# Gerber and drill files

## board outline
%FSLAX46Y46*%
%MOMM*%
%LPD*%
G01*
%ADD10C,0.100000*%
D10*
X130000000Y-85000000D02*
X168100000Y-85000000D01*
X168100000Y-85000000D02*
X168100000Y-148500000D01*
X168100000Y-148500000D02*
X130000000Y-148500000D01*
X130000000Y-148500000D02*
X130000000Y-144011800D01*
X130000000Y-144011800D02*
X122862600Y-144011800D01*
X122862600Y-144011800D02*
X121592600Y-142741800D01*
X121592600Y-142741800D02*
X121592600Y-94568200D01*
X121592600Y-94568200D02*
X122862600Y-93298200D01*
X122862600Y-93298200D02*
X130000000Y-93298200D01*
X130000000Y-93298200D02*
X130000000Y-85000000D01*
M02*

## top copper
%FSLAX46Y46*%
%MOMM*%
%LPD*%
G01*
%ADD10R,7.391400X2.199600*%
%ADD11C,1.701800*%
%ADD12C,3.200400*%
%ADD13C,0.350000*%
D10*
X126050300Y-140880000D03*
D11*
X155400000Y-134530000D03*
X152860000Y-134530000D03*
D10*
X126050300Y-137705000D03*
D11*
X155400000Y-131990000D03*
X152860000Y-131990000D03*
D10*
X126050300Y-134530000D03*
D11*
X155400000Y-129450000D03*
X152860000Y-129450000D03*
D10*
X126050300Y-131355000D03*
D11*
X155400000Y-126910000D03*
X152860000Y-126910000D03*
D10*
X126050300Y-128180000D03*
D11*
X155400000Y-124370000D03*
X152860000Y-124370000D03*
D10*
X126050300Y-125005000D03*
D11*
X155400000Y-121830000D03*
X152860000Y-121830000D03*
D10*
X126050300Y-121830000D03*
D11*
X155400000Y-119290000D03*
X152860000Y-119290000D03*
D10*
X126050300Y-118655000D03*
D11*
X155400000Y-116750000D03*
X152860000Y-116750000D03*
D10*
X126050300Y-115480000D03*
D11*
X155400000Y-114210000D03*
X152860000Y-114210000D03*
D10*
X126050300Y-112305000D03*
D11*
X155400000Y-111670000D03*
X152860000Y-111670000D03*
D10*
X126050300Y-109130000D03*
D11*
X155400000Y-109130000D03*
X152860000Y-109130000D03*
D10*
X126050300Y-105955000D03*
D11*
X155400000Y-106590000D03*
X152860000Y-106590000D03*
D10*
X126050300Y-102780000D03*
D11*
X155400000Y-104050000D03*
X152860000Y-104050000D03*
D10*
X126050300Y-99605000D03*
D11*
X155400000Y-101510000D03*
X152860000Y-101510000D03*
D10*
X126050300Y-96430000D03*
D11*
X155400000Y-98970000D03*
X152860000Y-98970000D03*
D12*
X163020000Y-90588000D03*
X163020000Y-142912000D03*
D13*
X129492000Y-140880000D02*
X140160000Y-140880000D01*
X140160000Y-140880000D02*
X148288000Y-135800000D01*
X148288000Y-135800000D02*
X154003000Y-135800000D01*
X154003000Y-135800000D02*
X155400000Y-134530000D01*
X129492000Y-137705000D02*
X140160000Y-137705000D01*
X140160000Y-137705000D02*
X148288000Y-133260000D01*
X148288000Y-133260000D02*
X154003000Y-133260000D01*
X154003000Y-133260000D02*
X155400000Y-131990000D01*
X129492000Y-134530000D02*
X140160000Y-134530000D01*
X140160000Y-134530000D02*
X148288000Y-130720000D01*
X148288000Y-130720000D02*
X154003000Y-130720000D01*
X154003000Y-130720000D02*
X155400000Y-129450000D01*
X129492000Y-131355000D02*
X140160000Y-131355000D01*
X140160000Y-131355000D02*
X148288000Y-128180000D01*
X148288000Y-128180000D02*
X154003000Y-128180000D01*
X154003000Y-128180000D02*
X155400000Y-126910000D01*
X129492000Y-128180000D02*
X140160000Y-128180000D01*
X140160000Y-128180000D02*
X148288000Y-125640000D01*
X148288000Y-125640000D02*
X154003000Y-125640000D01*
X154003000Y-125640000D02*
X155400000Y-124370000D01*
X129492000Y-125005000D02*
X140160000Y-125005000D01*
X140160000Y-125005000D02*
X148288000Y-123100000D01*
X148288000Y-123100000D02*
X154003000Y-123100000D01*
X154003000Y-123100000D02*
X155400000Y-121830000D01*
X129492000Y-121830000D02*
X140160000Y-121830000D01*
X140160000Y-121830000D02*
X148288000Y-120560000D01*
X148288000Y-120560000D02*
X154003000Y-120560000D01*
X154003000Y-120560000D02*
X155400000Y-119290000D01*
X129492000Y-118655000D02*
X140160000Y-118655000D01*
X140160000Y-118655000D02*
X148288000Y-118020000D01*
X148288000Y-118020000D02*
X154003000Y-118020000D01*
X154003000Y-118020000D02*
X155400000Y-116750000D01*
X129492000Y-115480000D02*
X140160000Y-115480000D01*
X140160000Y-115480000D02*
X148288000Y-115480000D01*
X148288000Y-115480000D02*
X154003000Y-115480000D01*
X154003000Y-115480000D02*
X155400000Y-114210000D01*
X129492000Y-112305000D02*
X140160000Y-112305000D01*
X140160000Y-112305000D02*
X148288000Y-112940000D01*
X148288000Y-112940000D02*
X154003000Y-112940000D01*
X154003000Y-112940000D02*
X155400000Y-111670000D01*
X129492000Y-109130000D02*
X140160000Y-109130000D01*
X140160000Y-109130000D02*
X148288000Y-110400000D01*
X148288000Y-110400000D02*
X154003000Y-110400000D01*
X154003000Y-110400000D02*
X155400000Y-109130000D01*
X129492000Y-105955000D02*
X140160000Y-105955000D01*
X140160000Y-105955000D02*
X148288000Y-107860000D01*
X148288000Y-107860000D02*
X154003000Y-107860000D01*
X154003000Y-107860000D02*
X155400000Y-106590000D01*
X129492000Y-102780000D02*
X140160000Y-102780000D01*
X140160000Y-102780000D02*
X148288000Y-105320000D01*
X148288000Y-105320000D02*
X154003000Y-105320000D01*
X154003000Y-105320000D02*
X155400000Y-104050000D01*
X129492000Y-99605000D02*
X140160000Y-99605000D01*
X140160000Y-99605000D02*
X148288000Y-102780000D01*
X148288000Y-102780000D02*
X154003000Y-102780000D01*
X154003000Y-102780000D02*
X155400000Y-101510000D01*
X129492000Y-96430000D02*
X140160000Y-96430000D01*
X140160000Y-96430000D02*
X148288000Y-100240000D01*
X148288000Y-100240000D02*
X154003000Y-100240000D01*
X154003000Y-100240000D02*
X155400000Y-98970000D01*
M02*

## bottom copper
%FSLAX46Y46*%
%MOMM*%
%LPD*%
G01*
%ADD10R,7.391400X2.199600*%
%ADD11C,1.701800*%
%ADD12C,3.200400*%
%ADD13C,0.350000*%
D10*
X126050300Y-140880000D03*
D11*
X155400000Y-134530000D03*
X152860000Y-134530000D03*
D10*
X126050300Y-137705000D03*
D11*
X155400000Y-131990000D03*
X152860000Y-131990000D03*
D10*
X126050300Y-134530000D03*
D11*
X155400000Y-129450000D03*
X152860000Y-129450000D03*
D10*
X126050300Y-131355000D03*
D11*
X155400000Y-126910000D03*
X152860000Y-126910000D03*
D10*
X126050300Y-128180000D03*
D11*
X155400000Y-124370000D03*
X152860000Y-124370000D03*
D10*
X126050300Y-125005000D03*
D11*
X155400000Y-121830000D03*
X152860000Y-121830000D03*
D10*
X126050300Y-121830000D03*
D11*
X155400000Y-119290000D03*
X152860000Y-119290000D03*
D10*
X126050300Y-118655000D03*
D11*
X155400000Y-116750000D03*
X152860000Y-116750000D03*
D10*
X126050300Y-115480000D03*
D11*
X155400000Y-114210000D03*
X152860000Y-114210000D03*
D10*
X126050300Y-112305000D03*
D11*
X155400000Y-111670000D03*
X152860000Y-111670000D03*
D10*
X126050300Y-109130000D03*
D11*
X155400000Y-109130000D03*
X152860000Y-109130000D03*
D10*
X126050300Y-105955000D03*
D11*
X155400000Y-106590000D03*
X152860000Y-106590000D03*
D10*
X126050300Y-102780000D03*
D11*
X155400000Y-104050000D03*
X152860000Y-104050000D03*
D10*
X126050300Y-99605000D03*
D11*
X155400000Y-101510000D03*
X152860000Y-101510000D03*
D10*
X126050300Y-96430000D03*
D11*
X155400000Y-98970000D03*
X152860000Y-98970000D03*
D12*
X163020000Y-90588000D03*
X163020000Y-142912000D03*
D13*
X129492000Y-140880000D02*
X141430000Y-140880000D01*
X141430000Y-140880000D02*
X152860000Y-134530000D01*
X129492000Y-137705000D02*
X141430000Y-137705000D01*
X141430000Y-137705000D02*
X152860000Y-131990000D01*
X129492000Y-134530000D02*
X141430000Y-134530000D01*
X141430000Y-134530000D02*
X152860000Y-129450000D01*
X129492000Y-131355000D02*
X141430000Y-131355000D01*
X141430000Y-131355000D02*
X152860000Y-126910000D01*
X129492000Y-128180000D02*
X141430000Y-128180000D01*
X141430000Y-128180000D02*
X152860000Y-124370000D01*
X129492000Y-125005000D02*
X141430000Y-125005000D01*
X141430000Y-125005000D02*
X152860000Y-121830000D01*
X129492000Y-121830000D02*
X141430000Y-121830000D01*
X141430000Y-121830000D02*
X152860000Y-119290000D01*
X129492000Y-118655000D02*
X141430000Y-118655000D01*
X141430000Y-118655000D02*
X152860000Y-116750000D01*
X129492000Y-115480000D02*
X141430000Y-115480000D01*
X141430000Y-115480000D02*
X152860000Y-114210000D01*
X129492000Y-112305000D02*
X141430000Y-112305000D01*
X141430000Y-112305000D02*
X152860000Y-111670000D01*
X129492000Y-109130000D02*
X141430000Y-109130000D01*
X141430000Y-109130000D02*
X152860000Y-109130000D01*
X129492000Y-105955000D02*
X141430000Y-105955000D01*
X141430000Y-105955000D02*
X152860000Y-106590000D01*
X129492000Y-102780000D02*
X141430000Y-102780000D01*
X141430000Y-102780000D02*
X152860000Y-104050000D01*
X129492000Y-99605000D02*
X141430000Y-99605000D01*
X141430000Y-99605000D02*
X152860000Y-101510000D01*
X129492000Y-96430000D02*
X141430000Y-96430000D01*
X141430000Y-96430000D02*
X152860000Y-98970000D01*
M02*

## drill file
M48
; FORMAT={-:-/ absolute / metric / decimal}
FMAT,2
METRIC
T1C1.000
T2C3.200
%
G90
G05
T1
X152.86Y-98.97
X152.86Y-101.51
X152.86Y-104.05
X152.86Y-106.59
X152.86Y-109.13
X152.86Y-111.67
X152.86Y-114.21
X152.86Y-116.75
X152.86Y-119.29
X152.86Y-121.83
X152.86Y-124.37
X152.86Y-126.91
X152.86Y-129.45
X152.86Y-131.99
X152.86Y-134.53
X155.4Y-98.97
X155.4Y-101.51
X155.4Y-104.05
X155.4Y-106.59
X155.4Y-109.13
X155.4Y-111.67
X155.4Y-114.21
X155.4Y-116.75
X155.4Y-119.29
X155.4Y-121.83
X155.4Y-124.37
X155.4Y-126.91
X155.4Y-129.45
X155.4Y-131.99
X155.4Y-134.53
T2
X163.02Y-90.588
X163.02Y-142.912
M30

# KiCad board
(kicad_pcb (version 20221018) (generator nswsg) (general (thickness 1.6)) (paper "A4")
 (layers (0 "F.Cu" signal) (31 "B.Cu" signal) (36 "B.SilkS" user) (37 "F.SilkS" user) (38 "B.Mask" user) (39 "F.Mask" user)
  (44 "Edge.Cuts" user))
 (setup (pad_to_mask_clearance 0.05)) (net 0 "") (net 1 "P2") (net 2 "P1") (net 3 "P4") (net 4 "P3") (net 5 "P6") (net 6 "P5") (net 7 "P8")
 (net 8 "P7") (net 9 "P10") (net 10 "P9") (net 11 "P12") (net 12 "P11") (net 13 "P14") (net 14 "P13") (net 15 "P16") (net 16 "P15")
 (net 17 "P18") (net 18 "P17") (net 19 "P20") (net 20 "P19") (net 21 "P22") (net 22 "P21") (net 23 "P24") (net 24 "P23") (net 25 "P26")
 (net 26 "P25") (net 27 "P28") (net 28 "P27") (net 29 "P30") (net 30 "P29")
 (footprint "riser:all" (layer "F.Cu") (at 130.0 85.0)
  (pad "2" smd rect (at -3.9497 55.88) (size 7.3914 2.1996) (layers "F.Cu" "F.Mask") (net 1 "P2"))
  (pad "1" smd rect (at -3.9497 55.88) (size 7.3914 2.1996) (layers "B.Cu" "B.Mask") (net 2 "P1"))
  (pad "2" thru_hole circle (at 25.4 49.53) (size 1.7018 1.7018) (drill 1.0) (layers "*.Cu" "*.Mask") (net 1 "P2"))
  (pad "1" thru_hole circle (at 22.86 49.53) (size 1.7018 1.7018) (drill 1.0) (layers "*.Cu" "*.Mask") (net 2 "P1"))
  (pad "4" smd rect (at -3.9497 52.705) (size 7.3914 2.1996) (layers "F.Cu" "F.Mask") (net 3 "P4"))
  (pad "3" smd rect (at -3.9497 52.705) (size 7.3914 2.1996) (layers "B.Cu" "B.Mask") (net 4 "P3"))
  (pad "4" thru_hole circle (at 25.4 46.99) (size 1.7018 1.7018) (drill 1.0) (layers "*.Cu" "*.Mask") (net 3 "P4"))
  (pad "3" thru_hole circle (at 22.86 46.99) (size 1.7018 1.7018) (drill 1.0) (layers "*.Cu" "*.Mask") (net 4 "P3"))
  (pad "6" smd rect (at -3.9497 49.53) (size 7.3914 2.1996) (layers "F.Cu" "F.Mask") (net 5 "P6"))
  (pad "5" smd rect (at -3.9497 49.53) (size 7.3914 2.1996) (layers "B.Cu" "B.Mask") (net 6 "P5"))
  (pad "6" thru_hole circle (at 25.4 44.45) (size 1.7018 1.7018) (drill 1.0) (layers "*.Cu" "*.Mask") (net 5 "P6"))
  (pad "5" thru_hole circle (at 22.86 44.45) (size 1.7018 1.7018) (drill 1.0) (layers "*.Cu" "*.Mask") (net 6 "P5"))
  (pad "8" smd rect (at -3.9497 46.355) (size 7.3914 2.1996) (layers "F.Cu" "F.Mask") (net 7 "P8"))
  (pad "7" smd rect (at -3.9497 46.355) (size 7.3914 2.1996) (layers "B.Cu" "B.Mask") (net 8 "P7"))
  (pad "8" thru_hole circle (at 25.4 41.91) (size 1.7018 1.7018) (drill 1.0) (layers "*.Cu" "*.Mask") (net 7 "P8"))
  (pad "7" thru_hole circle (at 22.86 41.91) (size 1.7018 1.7018) (drill 1.0) (layers "*.Cu" "*.Mask") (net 8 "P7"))
  (pad "10" smd rect (at -3.9497 43.18) (size 7.3914 2.1996) (layers "F.Cu" "F.Mask") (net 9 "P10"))
  (pad "9" smd rect (at -3.9497 43.18) (size 7.3914 2.1996) (layers "B.Cu" "B.Mask") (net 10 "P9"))
  (pad "10" thru_hole circle (at 25.4 39.37) (size 1.7018 1.7018) (drill 1.0) (layers "*.Cu" "*.Mask") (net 9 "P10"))
  (pad "9" thru_hole circle (at 22.86 39.37) (size 1.7018 1.7018) (drill 1.0) (layers "*.Cu" "*.Mask") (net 10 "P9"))
  (pad "12" smd rect (at -3.9497 40.005) (size 7.3914 2.1996) (layers "F.Cu" "F.Mask") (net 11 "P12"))
  (pad "11" smd rect (at -3.9497 40.005) (size 7.3914 2.1996) (layers "B.Cu" "B.Mask") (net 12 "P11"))
  (pad "12" thru_hole circle (at 25.4 36.83) (size 1.7018 1.7018) (drill 1.0) (layers "*.Cu" "*.Mask") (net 11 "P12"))
  (pad "11" thru_hole circle (at 22.86 36.83) (size 1.7018 1.7018) (drill 1.0) (layers "*.Cu" "*.Mask") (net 12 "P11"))
  (pad "14" smd rect (at -3.9497 36.83) (size 7.3914 2.1996) (layers "F.Cu" "F.Mask") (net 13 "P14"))
  (pad "13" smd rect (at -3.9497 36.83) (size 7.3914 2.1996) (layers "B.Cu" "B.Mask") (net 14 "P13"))
  (pad "14" thru_hole circle (at 25.4 34.29) (size 1.7018 1.7018) (drill 1.0) (layers "*.Cu" "*.Mask") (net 13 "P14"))
  (pad "13" thru_hole circle (at 22.86 34.29) (size 1.7018 1.7018) (drill 1.0) (layers "*.Cu" "*.Mask") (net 14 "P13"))
  (pad "16" smd rect (at -3.9497 33.655) (size 7.3914 2.1996) (layers "F.Cu" "F.Mask") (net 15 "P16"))
  (pad "15" smd rect (at -3.9497 33.655) (size 7.3914 2.1996) (layers "B.Cu" "B.Mask") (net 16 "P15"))
  (pad "16" thru_hole circle (at 25.4 31.75) (size 1.7018 1.7018) (drill 1.0) (layers "*.Cu" "*.Mask") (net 15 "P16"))
  (pad "15" thru_hole circle (at 22.86 31.75) (size 1.7018 1.7018) (drill 1.0) (layers "*.Cu" "*.Mask") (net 16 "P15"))
  (pad "18" smd rect (at -3.9497 30.48) (size 7.3914 2.1996) (layers "F.Cu" "F.Mask") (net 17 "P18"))
  (pad "17" smd rect (at -3.9497 30.48) (size 7.3914 2.1996) (layers "B.Cu" "B.Mask") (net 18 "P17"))
  (pad "18" thru_hole circle (at 25.4 29.21) (size 1.7018 1.7018) (drill 1.0) (layers "*.Cu" "*.Mask") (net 17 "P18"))
  (pad "17" thru_hole circle (at 22.86 29.21) (size 1.7018 1.7018) (drill 1.0) (layers "*.Cu" "*.Mask") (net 18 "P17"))
  (pad "20" smd rect (at -3.9497 27.305) (size 7.3914 2.1996) (layers "F.Cu" "F.Mask") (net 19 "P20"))
  (pad "19" smd rect (at -3.9497 27.305) (size 7.3914 2.1996) (layers "B.Cu" "B.Mask") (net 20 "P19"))
  (pad "20" thru_hole circle (at 25.4 26.67) (size 1.7018 1.7018) (drill 1.0) (layers "*.Cu" "*.Mask") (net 19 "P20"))
  (pad "19" thru_hole circle (at 22.86 26.67) (size 1.7018 1.7018) (drill 1.0) (layers "*.Cu" "*.Mask") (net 20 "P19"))
  (pad "22" smd rect (at -3.9497 24.13) (size 7.3914 2.1996) (layers "F.Cu" "F.Mask") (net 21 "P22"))
  (pad "21" smd rect (at -3.9497 24.13) (size 7.3914 2.1996) (layers "B.Cu" "B.Mask") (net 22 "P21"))
  (pad "22" thru_hole circle (at 25.4 24.13) (size 1.7018 1.7018) (drill 1.0) (layers "*.Cu" "*.Mask") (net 21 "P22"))
  (pad "21" thru_hole circle (at 22.86 24.13) (size 1.7018 1.7018) (drill 1.0) (layers "*.Cu" "*.Mask") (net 22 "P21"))
  (pad "24" smd rect (at -3.9497 20.955) (size 7.3914 2.1996) (layers "F.Cu" "F.Mask") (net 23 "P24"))
  (pad "23" smd rect (at -3.9497 20.955) (size 7.3914 2.1996) (layers "B.Cu" "B.Mask") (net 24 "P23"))
  (pad "24" thru_hole circle (at 25.4 21.59) (size 1.7018 1.7018) (drill 1.0) (layers "*.Cu" "*.Mask") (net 23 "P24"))
  (pad "23" thru_hole circle (at 22.86 21.59) (size 1.7018 1.7018) (drill 1.0) (layers "*.Cu" "*.Mask") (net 24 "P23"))
  (pad "26" smd rect (at -3.9497 17.78) (size 7.3914 2.1996) (layers "F.Cu" "F.Mask") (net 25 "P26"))
  (pad "25" smd rect (at -3.9497 17.78) (size 7.3914 2.1996) (layers "B.Cu" "B.Mask") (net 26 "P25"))
  (pad "26" thru_hole circle (at 25.4 19.05) (size 1.7018 1.7018) (drill 1.0) (layers "*.Cu" "*.Mask") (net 25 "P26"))
  (pad "25" thru_hole circle (at 22.86 19.05) (size 1.7018 1.7018) (drill 1.0) (layers "*.Cu" "*.Mask") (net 26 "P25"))
  (pad "28" smd rect (at -3.9497 14.605) (size 7.3914 2.1996) (layers "F.Cu" "F.Mask") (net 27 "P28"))
  (pad "27" smd rect (at -3.9497 14.605) (size 7.3914 2.1996) (layers "B.Cu" "B.Mask") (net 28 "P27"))
  (pad "28" thru_hole circle (at 25.4 16.51) (size 1.7018 1.7018) (drill 1.0) (layers "*.Cu" "*.Mask") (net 27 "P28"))
  (pad "27" thru_hole circle (at 22.86 16.51) (size 1.7018 1.7018) (drill 1.0) (layers "*.Cu" "*.Mask") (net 28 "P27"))
  (pad "30" smd rect (at -3.9497 11.43) (size 7.3914 2.1996) (layers "F.Cu" "F.Mask") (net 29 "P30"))
  (pad "29" smd rect (at -3.9497 11.43) (size 7.3914 2.1996) (layers "B.Cu" "B.Mask") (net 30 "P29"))
  (pad "30" thru_hole circle (at 25.4 13.97) (size 1.7018 1.7018) (drill 1.0) (layers "*.Cu" "*.Mask") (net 29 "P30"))
  (pad "29" thru_hole circle (at 22.86 13.97) (size 1.7018 1.7018) (drill 1.0) (layers "*.Cu" "*.Mask") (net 30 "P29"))
  (pad "" np_thru_hole circle (at 33.02 5.588) (size 3.2004 3.2004) (drill 3.2) (layers "*.Cu" "*.Mask"))
  (pad "" np_thru_hole circle (at 33.02 57.912) (size 3.2004 3.2004) (drill 3.2) (layers "*.Cu" "*.Mask")))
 (gr_line (start 130.0000 85.0000) (end 168.1000 85.0000) (layer "Edge.Cuts") (width 0.1))
 (gr_line (start 168.1000 85.0000) (end 168.1000 148.5000) (layer "Edge.Cuts") (width 0.1))
 (gr_line (start 168.1000 148.5000) (end 130.0000 148.5000) (layer "Edge.Cuts") (width 0.1))
 (gr_line (start 130.0000 148.5000) (end 130.0000 144.0118) (layer "Edge.Cuts") (width 0.1))
 (gr_line (start 130.0000 144.0118) (end 122.8626 144.0118) (layer "Edge.Cuts") (width 0.1))
 (gr_line (start 122.8626 144.0118) (end 121.5926 142.7418) (layer "Edge.Cuts") (width 0.1))
 (gr_line (start 121.5926 142.7418) (end 121.5926 94.5682) (layer "Edge.Cuts") (width 0.1))
 (gr_line (start 121.5926 94.5682) (end 122.8626 93.2982) (layer "Edge.Cuts") (width 0.1))
 (gr_line (start 122.8626 93.2982) (end 130.0000 93.2982) (layer "Edge.Cuts") (width 0.1))
 (gr_line (start 130.0000 93.2982) (end 130.0000 85.0000) (layer "Edge.Cuts") (width 0.1))
 (segment (start 129.4920 140.8800) (end 140.1600 140.8800) (width 0.35) (layer "F.Cu") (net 1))
 (segment (start 140.1600 140.8800) (end 148.2880 135.8000) (width 0.35) (layer "F.Cu") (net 1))
 (segment (start 148.2880 135.8000) (end 154.0030 135.8000) (width 0.35) (layer "F.Cu") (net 1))
 (segment (start 154.0030 135.8000) (end 155.4000 134.5300) (width 0.35) (layer "F.Cu") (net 1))
 (segment (start 129.4920 140.8800) (end 141.4300 140.8800) (width 0.35) (layer "B.Cu") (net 2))
 (segment (start 141.4300 140.8800) (end 152.8600 134.5300) (width 0.35) (layer "B.Cu") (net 2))
 (segment (start 129.4920 137.7050) (end 140.1600 137.7050) (width 0.35) (layer "F.Cu") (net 3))
 (segment (start 140.1600 137.7050) (end 148.2880 133.2600) (width 0.35) (layer "F.Cu") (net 3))
 (segment (start 148.2880 133.2600) (end 154.0030 133.2600) (width 0.35) (layer "F.Cu") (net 3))
 (segment (start 154.0030 133.2600) (end 155.4000 131.9900) (width 0.35) (layer "F.Cu") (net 3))
 (segment (start 129.4920 137.7050) (end 141.4300 137.7050) (width 0.35) (layer "B.Cu") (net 4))
 (segment (start 141.4300 137.7050) (end 152.8600 131.9900) (width 0.35) (layer "B.Cu") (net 4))
 (segment (start 129.4920 134.5300) (end 140.1600 134.5300) (width 0.35) (layer "F.Cu") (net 5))
 (segment (start 140.1600 134.5300) (end 148.2880 130.7200) (width 0.35) (layer "F.Cu") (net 5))
 (segment (start 148.2880 130.7200) (end 154.0030 130.7200) (width 0.35) (layer "F.Cu") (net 5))
 (segment (start 154.0030 130.7200) (end 155.4000 129.4500) (width 0.35) (layer "F.Cu") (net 5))
 (segment (start 129.4920 134.5300) (end 141.4300 134.5300) (width 0.35) (layer "B.Cu") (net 6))
 (segment (start 141.4300 134.5300) (end 152.8600 129.4500) (width 0.35) (layer "B.Cu") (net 6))
 (segment (start 129.4920 131.3550) (end 140.1600 131.3550) (width 0.35) (layer "F.Cu") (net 7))
 (segment (start 140.1600 131.3550) (end 148.2880 128.1800) (width 0.35) (layer "F.Cu") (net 7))
 (segment (start 148.2880 128.1800) (end 154.0030 128.1800) (width 0.35) (layer "F.Cu") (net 7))
 (segment (start 154.0030 128.1800) (end 155.4000 126.9100) (width 0.35) (layer "F.Cu") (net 7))
 (segment (start 129.4920 131.3550) (end 141.4300 131.3550) (width 0.35) (layer "B.Cu") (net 8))
 (segment (start 141.4300 131.3550) (end 152.8600 126.9100) (width 0.35) (layer "B.Cu") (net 8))
 (segment (start 129.4920 128.1800) (end 140.1600 128.1800) (width 0.35) (layer "F.Cu") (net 9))
 (segment (start 140.1600 128.1800) (end 148.2880 125.6400) (width 0.35) (layer "F.Cu") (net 9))
 (segment (start 148.2880 125.6400) (end 154.0030 125.6400) (width 0.35) (layer "F.Cu") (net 9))
 (segment (start 154.0030 125.6400) (end 155.4000 124.3700) (width 0.35) (layer "F.Cu") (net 9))
 (segment (start 129.4920 128.1800) (end 141.4300 128.1800) (width 0.35) (layer "B.Cu") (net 10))
 (segment (start 141.4300 128.1800) (end 152.8600 124.3700) (width 0.35) (layer "B.Cu") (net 10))
 (segment (start 129.4920 125.0050) (end 140.1600 125.0050) (width 0.35) (layer "F.Cu") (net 11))
 (segment (start 140.1600 125.0050) (end 148.2880 123.1000) (width 0.35) (layer "F.Cu") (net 11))
 (segment (start 148.2880 123.1000) (end 154.0030 123.1000) (width 0.35) (layer "F.Cu") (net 11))
 (segment (start 154.0030 123.1000) (end 155.4000 121.8300) (width 0.35) (layer "F.Cu") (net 11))
 (segment (start 129.4920 125.0050) (end 141.4300 125.0050) (width 0.35) (layer "B.Cu") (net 12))
 (segment (start 141.4300 125.0050) (end 152.8600 121.8300) (width 0.35) (layer "B.Cu") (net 12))
 (segment (start 129.4920 121.8300) (end 140.1600 121.8300) (width 0.35) (layer "F.Cu") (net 13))
 (segment (start 140.1600 121.8300) (end 148.2880 120.5600) (width 0.35) (layer "F.Cu") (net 13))
 (segment (start 148.2880 120.5600) (end 154.0030 120.5600) (width 0.35) (layer "F.Cu") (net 13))
 (segment (start 154.0030 120.5600) (end 155.4000 119.2900) (width 0.35) (layer "F.Cu") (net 13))
 (segment (start 129.4920 121.8300) (end 141.4300 121.8300) (width 0.35) (layer "B.Cu") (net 14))
 (segment (start 141.4300 121.8300) (end 152.8600 119.2900) (width 0.35) (layer "B.Cu") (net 14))
 (segment (start 129.4920 118.6550) (end 140.1600 118.6550) (width 0.35) (layer "F.Cu") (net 15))
 (segment (start 140.1600 118.6550) (end 148.2880 118.0200) (width 0.35) (layer "F.Cu") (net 15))
 (segment (start 148.2880 118.0200) (end 154.0030 118.0200) (width 0.35) (layer "F.Cu") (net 15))
 (segment (start 154.0030 118.0200) (end 155.4000 116.7500) (width 0.35) (layer "F.Cu") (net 15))
 (segment (start 129.4920 118.6550) (end 141.4300 118.6550) (width 0.35) (layer "B.Cu") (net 16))
 (segment (start 141.4300 118.6550) (end 152.8600 116.7500) (width 0.35) (layer "B.Cu") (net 16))
 (segment (start 129.4920 115.4800) (end 140.1600 115.4800) (width 0.35) (layer "F.Cu") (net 17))
 (segment (start 140.1600 115.4800) (end 148.2880 115.4800) (width 0.35) (layer "F.Cu") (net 17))
 (segment (start 148.2880 115.4800) (end 154.0030 115.4800) (width 0.35) (layer "F.Cu") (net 17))
 (segment (start 154.0030 115.4800) (end 155.4000 114.2100) (width 0.35) (layer "F.Cu") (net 17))
 (segment (start 129.4920 115.4800) (end 141.4300 115.4800) (width 0.35) (layer "B.Cu") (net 18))
 (segment (start 141.4300 115.4800) (end 152.8600 114.2100) (width 0.35) (layer "B.Cu") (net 18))
 (segment (start 129.4920 112.3050) (end 140.1600 112.3050) (width 0.35) (layer "F.Cu") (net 19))
 (segment (start 140.1600 112.3050) (end 148.2880 112.9400) (width 0.35) (layer "F.Cu") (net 19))
 (segment (start 148.2880 112.9400) (end 154.0030 112.9400) (width 0.35) (layer "F.Cu") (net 19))
 (segment (start 154.0030 112.9400) (end 155.4000 111.6700) (width 0.35) (layer "F.Cu") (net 19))
 (segment (start 129.4920 112.3050) (end 141.4300 112.3050) (width 0.35) (layer "B.Cu") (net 20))
 (segment (start 141.4300 112.3050) (end 152.8600 111.6700) (width 0.35) (layer "B.Cu") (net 20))
 (segment (start 129.4920 109.1300) (end 140.1600 109.1300) (width 0.35) (layer "F.Cu") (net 21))
 (segment (start 140.1600 109.1300) (end 148.2880 110.4000) (width 0.35) (layer "F.Cu") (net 21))
 (segment (start 148.2880 110.4000) (end 154.0030 110.4000) (width 0.35) (layer "F.Cu") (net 21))
 (segment (start 154.0030 110.4000) (end 155.4000 109.1300) (width 0.35) (layer "F.Cu") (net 21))
 (segment (start 129.4920 109.1300) (end 141.4300 109.1300) (width 0.35) (layer "B.Cu") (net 22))
 (segment (start 141.4300 109.1300) (end 152.8600 109.1300) (width 0.35) (layer "B.Cu") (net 22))
 (segment (start 129.4920 105.9550) (end 140.1600 105.9550) (width 0.35) (layer "F.Cu") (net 23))
 (segment (start 140.1600 105.9550) (end 148.2880 107.8600) (width 0.35) (layer "F.Cu") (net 23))
 (segment (start 148.2880 107.8600) (end 154.0030 107.8600) (width 0.35) (layer "F.Cu") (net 23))
 (segment (start 154.0030 107.8600) (end 155.4000 106.5900) (width 0.35) (layer "F.Cu") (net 23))
 (segment (start 129.4920 105.9550) (end 141.4300 105.9550) (width 0.35) (layer "B.Cu") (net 24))
 (segment (start 141.4300 105.9550) (end 152.8600 106.5900) (width 0.35) (layer "B.Cu") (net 24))
 (segment (start 129.4920 102.7800) (end 140.1600 102.7800) (width 0.35) (layer "F.Cu") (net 25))
 (segment (start 140.1600 102.7800) (end 148.2880 105.3200) (width 0.35) (layer "F.Cu") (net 25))
 (segment (start 148.2880 105.3200) (end 154.0030 105.3200) (width 0.35) (layer "F.Cu") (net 25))
 (segment (start 154.0030 105.3200) (end 155.4000 104.0500) (width 0.35) (layer "F.Cu") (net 25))
 (segment (start 129.4920 102.7800) (end 141.4300 102.7800) (width 0.35) (layer "B.Cu") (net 26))
 (segment (start 141.4300 102.7800) (end 152.8600 104.0500) (width 0.35) (layer "B.Cu") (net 26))
 (segment (start 129.4920 99.6050) (end 140.1600 99.6050) (width 0.35) (layer "F.Cu") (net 27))
 (segment (start 140.1600 99.6050) (end 148.2880 102.7800) (width 0.35) (layer "F.Cu") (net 27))
 (segment (start 148.2880 102.7800) (end 154.0030 102.7800) (width 0.35) (layer "F.Cu") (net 27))
 (segment (start 154.0030 102.7800) (end 155.4000 101.5100) (width 0.35) (layer "F.Cu") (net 27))
 (segment (start 129.4920 99.6050) (end 141.4300 99.6050) (width 0.35) (layer "B.Cu") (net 28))
 (segment (start 141.4300 99.6050) (end 152.8600 101.5100) (width 0.35) (layer "B.Cu") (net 28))
 (segment (start 129.4920 96.4300) (end 140.1600 96.4300) (width 0.35) (layer "F.Cu") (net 29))
 (segment (start 140.1600 96.4300) (end 148.2880 100.2400) (width 0.35) (layer "F.Cu") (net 29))
 (segment (start 148.2880 100.2400) (end 154.0030 100.2400) (width 0.35) (layer "F.Cu") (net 29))
 (segment (start 154.0030 100.2400) (end 155.4000 98.9700) (width 0.35) (layer "F.Cu") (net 29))
 (segment (start 129.4920 96.4300) (end 141.4300 96.4300) (width 0.35) (layer "B.Cu") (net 30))
 (segment (start 141.4300 96.4300) (end 152.8600 98.9700) (width 0.35) (layer "B.Cu") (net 30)))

